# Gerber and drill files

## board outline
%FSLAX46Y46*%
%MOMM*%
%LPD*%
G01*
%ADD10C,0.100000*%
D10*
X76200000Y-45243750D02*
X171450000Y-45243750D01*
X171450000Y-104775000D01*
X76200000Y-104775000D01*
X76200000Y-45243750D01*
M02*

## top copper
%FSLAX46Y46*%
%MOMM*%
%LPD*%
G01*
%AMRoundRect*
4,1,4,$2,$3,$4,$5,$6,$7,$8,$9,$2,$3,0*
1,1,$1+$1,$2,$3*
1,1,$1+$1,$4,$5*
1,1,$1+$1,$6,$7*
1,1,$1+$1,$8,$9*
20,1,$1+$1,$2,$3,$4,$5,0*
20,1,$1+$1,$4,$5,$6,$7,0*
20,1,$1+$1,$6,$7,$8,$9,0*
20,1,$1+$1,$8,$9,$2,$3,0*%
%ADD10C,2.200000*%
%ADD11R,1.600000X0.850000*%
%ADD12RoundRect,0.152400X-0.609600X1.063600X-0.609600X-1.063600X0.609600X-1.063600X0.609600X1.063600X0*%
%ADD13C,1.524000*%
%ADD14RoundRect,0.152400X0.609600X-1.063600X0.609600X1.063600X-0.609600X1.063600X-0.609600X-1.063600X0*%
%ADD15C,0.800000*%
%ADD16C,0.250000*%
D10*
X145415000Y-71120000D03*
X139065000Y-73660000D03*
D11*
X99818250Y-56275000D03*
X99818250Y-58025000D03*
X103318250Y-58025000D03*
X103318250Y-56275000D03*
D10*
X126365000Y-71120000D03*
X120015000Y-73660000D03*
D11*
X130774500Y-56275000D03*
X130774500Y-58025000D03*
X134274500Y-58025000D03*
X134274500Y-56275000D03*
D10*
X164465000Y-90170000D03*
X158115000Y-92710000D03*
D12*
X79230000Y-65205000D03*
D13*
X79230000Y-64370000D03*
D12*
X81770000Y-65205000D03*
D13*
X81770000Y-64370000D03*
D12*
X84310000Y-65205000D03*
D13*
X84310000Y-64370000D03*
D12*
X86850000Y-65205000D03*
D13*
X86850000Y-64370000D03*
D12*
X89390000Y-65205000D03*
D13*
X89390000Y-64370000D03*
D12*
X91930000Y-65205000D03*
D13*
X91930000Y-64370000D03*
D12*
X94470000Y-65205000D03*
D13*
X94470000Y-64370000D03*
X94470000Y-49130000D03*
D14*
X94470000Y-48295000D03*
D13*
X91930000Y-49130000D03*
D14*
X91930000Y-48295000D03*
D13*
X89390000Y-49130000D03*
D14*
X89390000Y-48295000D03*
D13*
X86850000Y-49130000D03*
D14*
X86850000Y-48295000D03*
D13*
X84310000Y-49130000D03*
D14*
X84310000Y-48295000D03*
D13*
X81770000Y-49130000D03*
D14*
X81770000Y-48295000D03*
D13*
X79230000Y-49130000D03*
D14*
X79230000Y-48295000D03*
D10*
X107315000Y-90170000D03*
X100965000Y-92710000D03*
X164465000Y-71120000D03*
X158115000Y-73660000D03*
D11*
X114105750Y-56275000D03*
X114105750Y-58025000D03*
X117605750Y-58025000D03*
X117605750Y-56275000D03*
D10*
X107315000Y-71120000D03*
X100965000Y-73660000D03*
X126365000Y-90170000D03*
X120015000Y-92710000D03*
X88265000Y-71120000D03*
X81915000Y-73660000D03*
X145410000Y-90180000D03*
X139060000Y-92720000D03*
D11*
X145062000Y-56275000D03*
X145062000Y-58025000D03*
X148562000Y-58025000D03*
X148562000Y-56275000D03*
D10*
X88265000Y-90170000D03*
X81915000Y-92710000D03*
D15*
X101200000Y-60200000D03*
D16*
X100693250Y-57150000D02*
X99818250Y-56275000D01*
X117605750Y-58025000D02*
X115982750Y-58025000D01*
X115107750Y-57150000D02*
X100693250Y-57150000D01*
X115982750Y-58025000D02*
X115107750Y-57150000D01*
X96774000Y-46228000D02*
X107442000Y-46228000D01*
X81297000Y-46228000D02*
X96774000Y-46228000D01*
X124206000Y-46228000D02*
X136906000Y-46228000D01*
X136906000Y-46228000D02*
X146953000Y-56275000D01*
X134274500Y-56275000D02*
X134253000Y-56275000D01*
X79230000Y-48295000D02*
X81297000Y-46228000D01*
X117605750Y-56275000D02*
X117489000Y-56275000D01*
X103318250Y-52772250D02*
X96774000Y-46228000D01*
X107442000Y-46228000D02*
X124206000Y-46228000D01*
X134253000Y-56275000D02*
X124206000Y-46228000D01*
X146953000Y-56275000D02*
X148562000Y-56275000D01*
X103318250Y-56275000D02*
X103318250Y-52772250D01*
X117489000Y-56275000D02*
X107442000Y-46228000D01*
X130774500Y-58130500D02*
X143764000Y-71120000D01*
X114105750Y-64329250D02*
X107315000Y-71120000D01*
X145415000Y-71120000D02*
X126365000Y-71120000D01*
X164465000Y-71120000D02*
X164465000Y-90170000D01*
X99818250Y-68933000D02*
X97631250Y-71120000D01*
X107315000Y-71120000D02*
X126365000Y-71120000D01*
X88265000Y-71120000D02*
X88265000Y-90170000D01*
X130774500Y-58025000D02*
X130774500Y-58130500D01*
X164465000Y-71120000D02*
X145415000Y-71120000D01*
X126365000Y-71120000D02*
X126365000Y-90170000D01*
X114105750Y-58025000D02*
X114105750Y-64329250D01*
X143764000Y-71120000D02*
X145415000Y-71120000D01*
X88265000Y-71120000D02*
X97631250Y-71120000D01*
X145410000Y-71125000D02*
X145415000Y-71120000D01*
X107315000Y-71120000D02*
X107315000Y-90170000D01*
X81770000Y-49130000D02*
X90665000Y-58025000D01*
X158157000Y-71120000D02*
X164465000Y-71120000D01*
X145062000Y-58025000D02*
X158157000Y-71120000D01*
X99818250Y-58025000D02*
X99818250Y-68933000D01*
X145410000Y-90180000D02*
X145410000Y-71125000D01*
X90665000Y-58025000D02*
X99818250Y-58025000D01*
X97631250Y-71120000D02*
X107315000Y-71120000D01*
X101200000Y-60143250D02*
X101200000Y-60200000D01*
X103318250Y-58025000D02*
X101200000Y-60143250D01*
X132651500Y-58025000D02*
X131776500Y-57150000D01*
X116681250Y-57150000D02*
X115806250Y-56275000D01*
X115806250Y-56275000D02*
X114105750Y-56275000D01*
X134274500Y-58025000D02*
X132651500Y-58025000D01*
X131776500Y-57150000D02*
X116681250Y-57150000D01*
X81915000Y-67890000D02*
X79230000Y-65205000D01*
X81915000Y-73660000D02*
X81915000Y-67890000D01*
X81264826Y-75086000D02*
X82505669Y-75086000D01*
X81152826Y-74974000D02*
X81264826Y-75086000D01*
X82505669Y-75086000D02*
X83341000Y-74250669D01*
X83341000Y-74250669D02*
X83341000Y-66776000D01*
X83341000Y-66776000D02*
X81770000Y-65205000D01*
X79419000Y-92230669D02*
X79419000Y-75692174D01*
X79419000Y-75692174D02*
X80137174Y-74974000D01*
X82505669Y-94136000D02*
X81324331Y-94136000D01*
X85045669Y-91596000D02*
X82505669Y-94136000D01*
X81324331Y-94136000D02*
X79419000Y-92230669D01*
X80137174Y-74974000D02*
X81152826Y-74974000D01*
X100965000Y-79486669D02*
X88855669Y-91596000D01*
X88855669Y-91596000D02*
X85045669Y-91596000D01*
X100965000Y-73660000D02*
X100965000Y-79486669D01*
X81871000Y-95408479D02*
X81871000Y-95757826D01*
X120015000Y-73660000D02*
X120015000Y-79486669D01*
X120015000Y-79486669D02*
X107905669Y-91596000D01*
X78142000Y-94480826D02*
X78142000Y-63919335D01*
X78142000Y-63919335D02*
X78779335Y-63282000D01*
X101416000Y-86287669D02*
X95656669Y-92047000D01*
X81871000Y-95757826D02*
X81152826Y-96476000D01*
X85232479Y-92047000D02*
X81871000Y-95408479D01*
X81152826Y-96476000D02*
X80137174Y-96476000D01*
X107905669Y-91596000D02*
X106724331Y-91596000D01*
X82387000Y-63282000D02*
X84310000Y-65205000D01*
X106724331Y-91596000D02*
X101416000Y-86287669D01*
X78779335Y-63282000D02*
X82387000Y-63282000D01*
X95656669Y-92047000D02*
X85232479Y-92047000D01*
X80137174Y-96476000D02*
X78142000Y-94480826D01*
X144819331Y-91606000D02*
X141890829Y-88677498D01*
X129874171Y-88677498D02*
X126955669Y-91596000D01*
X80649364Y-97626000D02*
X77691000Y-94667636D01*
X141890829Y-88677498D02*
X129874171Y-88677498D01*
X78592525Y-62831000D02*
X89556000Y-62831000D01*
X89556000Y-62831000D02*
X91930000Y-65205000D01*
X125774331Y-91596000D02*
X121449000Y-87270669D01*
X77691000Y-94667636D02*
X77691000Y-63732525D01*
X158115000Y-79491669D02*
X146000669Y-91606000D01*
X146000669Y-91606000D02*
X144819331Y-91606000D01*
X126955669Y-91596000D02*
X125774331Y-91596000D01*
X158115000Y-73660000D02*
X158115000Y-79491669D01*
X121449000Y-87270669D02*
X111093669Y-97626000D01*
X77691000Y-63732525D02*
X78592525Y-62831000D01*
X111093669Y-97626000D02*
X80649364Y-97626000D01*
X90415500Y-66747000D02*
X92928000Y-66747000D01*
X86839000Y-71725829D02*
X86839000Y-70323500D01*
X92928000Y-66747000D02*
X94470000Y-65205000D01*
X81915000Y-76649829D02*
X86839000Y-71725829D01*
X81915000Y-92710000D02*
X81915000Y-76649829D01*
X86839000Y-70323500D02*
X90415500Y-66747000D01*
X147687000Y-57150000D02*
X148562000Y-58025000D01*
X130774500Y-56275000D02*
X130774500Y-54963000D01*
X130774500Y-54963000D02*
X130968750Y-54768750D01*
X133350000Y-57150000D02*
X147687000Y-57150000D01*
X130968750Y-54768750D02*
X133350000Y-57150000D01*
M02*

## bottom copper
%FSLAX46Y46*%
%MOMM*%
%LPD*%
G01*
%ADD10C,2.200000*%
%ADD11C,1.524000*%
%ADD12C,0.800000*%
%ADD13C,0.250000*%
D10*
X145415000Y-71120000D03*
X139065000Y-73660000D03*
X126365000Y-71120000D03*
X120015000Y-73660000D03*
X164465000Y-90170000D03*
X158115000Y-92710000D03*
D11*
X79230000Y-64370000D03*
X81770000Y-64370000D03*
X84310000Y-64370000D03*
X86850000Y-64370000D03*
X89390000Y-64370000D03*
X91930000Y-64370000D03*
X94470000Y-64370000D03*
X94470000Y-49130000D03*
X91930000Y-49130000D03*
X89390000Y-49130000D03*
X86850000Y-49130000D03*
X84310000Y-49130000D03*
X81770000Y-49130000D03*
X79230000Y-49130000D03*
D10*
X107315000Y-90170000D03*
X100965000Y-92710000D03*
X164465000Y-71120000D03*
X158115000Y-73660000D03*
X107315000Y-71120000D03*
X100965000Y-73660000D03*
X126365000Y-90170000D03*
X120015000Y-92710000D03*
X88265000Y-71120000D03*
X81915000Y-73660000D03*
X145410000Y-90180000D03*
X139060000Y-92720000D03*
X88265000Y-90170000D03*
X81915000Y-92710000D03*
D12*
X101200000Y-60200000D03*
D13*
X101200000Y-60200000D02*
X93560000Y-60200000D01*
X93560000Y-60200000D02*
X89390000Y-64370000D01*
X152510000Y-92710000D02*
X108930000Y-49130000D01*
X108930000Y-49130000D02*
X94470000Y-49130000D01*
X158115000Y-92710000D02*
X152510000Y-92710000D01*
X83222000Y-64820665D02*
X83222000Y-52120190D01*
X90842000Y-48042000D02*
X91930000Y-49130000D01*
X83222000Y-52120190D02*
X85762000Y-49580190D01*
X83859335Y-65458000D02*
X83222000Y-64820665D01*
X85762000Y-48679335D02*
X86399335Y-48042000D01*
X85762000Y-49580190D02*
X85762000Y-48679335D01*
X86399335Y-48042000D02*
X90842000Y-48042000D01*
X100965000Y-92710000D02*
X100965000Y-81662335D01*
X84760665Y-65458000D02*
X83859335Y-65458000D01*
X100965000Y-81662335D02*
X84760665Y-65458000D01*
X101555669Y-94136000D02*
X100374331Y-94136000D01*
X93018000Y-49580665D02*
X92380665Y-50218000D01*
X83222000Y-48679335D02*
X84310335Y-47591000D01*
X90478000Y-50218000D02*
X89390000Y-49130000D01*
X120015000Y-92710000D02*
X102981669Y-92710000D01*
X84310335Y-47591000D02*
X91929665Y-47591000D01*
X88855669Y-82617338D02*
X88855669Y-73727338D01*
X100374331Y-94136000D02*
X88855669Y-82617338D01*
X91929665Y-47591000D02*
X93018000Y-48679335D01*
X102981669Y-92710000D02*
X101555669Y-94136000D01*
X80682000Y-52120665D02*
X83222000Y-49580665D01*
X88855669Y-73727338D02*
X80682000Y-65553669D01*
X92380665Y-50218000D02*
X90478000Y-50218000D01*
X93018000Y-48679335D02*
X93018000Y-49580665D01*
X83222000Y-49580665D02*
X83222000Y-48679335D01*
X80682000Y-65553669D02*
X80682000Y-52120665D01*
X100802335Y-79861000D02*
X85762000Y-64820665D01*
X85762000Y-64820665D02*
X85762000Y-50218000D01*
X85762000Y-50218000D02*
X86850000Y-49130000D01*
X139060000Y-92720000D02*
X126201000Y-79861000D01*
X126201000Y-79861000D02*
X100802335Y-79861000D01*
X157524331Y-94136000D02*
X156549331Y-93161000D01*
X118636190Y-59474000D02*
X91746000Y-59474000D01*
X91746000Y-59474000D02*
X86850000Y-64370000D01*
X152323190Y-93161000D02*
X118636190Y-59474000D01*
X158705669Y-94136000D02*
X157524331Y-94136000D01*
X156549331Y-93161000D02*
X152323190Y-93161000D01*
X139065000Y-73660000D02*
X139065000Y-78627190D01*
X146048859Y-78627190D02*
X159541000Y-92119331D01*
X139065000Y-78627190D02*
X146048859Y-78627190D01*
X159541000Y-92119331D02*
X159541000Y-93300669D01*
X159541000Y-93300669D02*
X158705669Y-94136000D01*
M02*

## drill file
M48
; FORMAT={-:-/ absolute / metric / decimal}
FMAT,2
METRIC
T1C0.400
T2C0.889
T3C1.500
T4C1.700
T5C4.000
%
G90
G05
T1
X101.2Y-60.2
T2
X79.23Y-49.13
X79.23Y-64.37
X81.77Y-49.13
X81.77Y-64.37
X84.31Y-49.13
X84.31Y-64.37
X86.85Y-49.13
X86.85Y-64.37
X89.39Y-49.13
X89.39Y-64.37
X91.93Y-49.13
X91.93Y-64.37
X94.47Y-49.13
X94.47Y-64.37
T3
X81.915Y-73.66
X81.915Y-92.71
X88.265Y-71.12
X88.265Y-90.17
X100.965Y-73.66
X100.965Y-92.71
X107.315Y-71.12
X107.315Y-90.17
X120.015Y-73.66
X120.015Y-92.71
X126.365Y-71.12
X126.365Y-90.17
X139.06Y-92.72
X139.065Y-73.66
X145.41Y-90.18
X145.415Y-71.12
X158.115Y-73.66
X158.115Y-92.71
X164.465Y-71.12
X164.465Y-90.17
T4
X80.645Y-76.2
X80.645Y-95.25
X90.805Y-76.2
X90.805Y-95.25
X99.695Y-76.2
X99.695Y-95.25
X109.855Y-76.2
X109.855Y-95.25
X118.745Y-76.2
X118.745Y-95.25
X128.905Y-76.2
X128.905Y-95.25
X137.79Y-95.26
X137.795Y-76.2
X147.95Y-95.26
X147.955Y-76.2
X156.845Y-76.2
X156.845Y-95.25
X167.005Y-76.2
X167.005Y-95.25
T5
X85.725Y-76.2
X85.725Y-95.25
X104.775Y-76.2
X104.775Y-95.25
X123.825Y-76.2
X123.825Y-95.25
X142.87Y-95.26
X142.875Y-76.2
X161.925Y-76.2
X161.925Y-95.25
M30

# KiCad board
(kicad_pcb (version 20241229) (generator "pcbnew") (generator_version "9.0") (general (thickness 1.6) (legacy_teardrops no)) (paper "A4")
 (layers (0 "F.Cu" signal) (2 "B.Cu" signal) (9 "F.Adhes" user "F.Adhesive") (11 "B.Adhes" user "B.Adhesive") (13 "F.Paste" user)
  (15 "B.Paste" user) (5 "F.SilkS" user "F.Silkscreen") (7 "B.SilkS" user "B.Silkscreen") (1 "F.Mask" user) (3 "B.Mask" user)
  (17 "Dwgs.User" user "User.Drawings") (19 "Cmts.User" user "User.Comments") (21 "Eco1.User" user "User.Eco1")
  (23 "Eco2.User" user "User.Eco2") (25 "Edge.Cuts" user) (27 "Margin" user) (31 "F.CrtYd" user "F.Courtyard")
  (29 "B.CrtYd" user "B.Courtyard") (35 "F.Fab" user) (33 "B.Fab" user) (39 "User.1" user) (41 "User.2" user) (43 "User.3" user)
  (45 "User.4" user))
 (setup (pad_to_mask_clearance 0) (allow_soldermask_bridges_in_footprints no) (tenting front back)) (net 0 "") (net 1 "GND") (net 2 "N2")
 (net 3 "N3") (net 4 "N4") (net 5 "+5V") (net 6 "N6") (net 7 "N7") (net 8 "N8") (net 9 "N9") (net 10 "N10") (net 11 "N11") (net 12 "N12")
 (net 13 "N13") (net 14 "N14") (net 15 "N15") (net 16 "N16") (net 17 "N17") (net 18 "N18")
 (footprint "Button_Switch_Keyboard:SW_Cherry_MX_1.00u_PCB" (layer "F.Cu") (at 145.415 71.12)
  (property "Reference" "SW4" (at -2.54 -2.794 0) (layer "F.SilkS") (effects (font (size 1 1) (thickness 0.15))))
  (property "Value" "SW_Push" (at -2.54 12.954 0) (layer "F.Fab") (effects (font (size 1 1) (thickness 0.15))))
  (pad "" np_thru_hole circle (at -7.62 5.08) (size 1.7 1.7) (drill 1.7) (layers "*.Cu" "*.Mask"))
  (pad "" np_thru_hole circle (at -2.54 5.08) (size 4 4) (drill 4) (layers "*.Cu" "*.Mask"))
  (pad "" np_thru_hole circle (at 2.54 5.08) (size 1.7 1.7) (drill 1.7) (layers "*.Cu" "*.Mask"))
  (pad "1" thru_hole circle (at 0 0) (size 2.2 2.2) (drill 1.5) (layers "*.Cu" "*.Mask") (remove_unused_layers no) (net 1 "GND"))
  (pad "2" thru_hole circle (at -6.35 2.54) (size 2.2 2.2) (drill 1.5) (layers "*.Cu" "*.Mask") (remove_unused_layers no) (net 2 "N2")))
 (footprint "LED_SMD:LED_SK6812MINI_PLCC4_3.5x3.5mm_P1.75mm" (layer "F.Cu") (at 101.56825 57.15)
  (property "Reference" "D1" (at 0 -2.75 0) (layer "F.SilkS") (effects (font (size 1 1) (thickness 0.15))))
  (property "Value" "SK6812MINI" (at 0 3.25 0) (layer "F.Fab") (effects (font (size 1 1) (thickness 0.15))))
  (pad "1" smd rect (at -1.75 -0.875) (size 1.6 0.85) (layers "F.Cu" "F.Mask" "F.Paste") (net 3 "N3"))
  (pad "2" smd rect (at -1.75 0.875) (size 1.6 0.85) (layers "F.Cu" "F.Mask" "F.Paste") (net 1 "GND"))
  (pad "3" smd rect (at 1.75 0.875) (size 1.6 0.85) (layers "F.Cu" "F.Mask" "F.Paste") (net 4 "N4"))
  (pad "4" smd rect (at 1.75 -0.875) (size 1.6 0.85) (layers "F.Cu" "F.Mask" "F.Paste") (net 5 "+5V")))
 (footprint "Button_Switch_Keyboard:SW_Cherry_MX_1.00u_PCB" (layer "F.Cu") (at 126.365 71.12)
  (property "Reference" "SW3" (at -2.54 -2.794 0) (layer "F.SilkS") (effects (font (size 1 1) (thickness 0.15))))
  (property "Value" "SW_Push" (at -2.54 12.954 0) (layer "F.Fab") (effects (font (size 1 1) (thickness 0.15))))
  (pad "" np_thru_hole circle (at -7.62 5.08) (size 1.7 1.7) (drill 1.7) (layers "*.Cu" "*.Mask"))
  (pad "" np_thru_hole circle (at -2.54 5.08) (size 4 4) (drill 4) (layers "*.Cu" "*.Mask"))
  (pad "" np_thru_hole circle (at 2.54 5.08) (size 1.7 1.7) (drill 1.7) (layers "*.Cu" "*.Mask"))
  (pad "1" thru_hole circle (at 0 0) (size 2.2 2.2) (drill 1.5) (layers "*.Cu" "*.Mask") (remove_unused_layers no) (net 1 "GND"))
  (pad "2" thru_hole circle (at -6.35 2.54) (size 2.2 2.2) (drill 1.5) (layers "*.Cu" "*.Mask") (remove_unused_layers no) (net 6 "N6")))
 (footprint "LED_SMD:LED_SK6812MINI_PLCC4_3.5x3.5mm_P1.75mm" (layer "F.Cu") (at 132.5245 57.15)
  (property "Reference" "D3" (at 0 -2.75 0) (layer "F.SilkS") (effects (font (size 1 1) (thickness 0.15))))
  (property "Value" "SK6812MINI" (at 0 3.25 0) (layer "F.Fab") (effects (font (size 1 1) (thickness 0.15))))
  (pad "1" smd rect (at -1.75 -0.875) (size 1.6 0.85) (layers "F.Cu" "F.Mask" "F.Paste") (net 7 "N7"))
  (pad "2" smd rect (at -1.75 0.875) (size 1.6 0.85) (layers "F.Cu" "F.Mask" "F.Paste") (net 1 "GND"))
  (pad "3" smd rect (at 1.75 0.875) (size 1.6 0.85) (layers "F.Cu" "F.Mask" "F.Paste") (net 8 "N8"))
  (pad "4" smd rect (at 1.75 -0.875) (size 1.6 0.85) (layers "F.Cu" "F.Mask" "F.Paste") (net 5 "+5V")))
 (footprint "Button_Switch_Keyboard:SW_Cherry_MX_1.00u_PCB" (layer "F.Cu") (at 164.465 90.17)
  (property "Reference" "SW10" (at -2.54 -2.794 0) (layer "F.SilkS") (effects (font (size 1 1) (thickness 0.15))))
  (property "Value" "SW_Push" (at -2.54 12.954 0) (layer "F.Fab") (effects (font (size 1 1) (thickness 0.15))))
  (pad "" np_thru_hole circle (at -7.62 5.08) (size 1.7 1.7) (drill 1.7) (layers "*.Cu" "*.Mask"))
  (pad "" np_thru_hole circle (at -2.54 5.08) (size 4 4) (drill 4) (layers "*.Cu" "*.Mask"))
  (pad "" np_thru_hole circle (at 2.54 5.08) (size 1.7 1.7) (drill 1.7) (layers "*.Cu" "*.Mask"))
  (pad "1" thru_hole circle (at 0 0) (size 2.2 2.2) (drill 1.5) (layers "*.Cu" "*.Mask") (remove_unused_layers no) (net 1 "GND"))
  (pad "2" thru_hole circle (at -6.35 2.54) (size 2.2 2.2) (drill 1.5) (layers "*.Cu" "*.Mask") (remove_unused_layers no) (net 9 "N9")))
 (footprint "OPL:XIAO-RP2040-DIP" (layer "F.Cu") (at 86.85 56.75 90)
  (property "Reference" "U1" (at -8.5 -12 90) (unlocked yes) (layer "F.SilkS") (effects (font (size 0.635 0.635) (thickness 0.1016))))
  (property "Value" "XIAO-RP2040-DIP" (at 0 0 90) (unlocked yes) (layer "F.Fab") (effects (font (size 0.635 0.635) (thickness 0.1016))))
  (pad "1" smd roundrect (at -8.455 -7.62 270) (size 2.432 1.524) (layers "F.Cu" "F.Mask") (roundrect_rratio 0.1) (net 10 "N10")
   (thermal_bridge_angle 45))
  (pad "1" thru_hole circle (at -7.62 -7.62 270) (size 1.524 1.524) (drill 0.889) (layers "*.Cu" "*.Mask") (remove_unused_layers no)
   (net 10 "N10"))
  (pad "2" smd roundrect (at -8.455 -5.08 270) (size 2.432 1.524) (layers "F.Cu" "F.Mask") (roundrect_rratio 0.1) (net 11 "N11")
   (thermal_bridge_angle 45))
  (pad "2" thru_hole circle (at -7.62 -5.08 270) (size 1.524 1.524) (drill 0.889) (layers "*.Cu" "*.Mask") (remove_unused_layers no)
   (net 11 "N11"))
  (pad "3" smd roundrect (at -8.455 -2.54 270) (size 2.432 1.524) (layers "F.Cu" "F.Mask") (roundrect_rratio 0.1) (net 6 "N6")
   (thermal_bridge_angle 45))
  (pad "3" thru_hole circle (at -7.62 -2.54 270) (size 1.524 1.524) (drill 0.889) (layers "*.Cu" "*.Mask") (remove_unused_layers no)
   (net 6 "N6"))
  (pad "4" smd roundrect (at -8.455 0 270) (size 2.432 1.524) (layers "F.Cu" "F.Mask") (roundrect_rratio 0.1) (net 2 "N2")
   (thermal_bridge_angle 45))
  (pad "4" thru_hole circle (at -7.62 0 270) (size 1.524 1.524) (drill 0.889) (layers "*.Cu" "*.Mask") (remove_unused_layers no)
   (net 2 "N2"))
  (pad "5" smd roundrect (at -8.455 2.54 270) (size 2.432 1.524) (layers "F.Cu" "F.Mask") (roundrect_rratio 0.1) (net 4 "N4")
   (thermal_bridge_angle 45))
  (pad "5" thru_hole circle (at -7.62 2.54 270) (size 1.524 1.524) (drill 0.889) (layers "*.Cu" "*.Mask") (remove_unused_layers no)
   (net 4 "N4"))
  (pad "6" smd roundrect (at -8.455 5.08 270) (size 2.432 1.524) (layers "F.Cu" "F.Mask") (roundrect_rratio 0.1) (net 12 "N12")
   (thermal_bridge_angle 45))
  (pad "6" thru_hole circle (at -7.62 5.08 270) (size 1.524 1.524) (drill 0.889) (layers "*.Cu" "*.Mask") (remove_unused_layers no)
   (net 12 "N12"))
  (pad "7" smd roundrect (at -8.455 7.62 270) (size 2.432 1.524) (layers "F.Cu" "F.Mask") (roundrect_rratio 0.1) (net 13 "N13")
   (thermal_bridge_angle 45))
  (pad "7" thru_hole circle (at -7.62 7.62 270) (size 1.524 1.524) (drill 0.889) (layers "*.Cu" "*.Mask") (remove_unused_layers no)
   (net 13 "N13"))
  (pad "8" thru_hole circle (at 7.62 7.62 90) (size 1.524 1.524) (drill 0.889) (layers "*.Cu" "*.Mask") (remove_unused_layers no)
   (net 9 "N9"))
  (pad "8" smd roundrect (at 8.455 7.62 90) (size 2.432 1.524) (layers "F.Cu" "F.Mask") (roundrect_rratio 0.1) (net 9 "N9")
   (thermal_bridge_angle 45))
  (pad "9" thru_hole circle (at 7.62 5.08 90) (size 1.524 1.524) (drill 0.889) (layers "*.Cu" "*.Mask") (remove_unused_layers no)
   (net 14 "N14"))
  (pad "9" smd roundrect (at 8.455 5.08 90) (size 2.432 1.524) (layers "F.Cu" "F.Mask") (roundrect_rratio 0.1) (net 14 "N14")
   (thermal_bridge_angle 45))
  (pad "10" thru_hole circle (at 7.62 2.54 90) (size 1.524 1.524) (drill 0.889) (layers "*.Cu" "*.Mask") (remove_unused_layers no)
   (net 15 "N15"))
  (pad "10" smd roundrect (at 8.455 2.54 90) (size 2.432 1.524) (layers "F.Cu" "F.Mask") (roundrect_rratio 0.1) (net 15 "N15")
   (thermal_bridge_angle 45))
  (pad "11" thru_hole circle (at 7.62 0 90) (size 1.524 1.524) (drill 0.889) (layers "*.Cu" "*.Mask") (remove_unused_layers no)
   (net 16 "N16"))
  (pad "11" smd roundrect (at 8.455 0 90) (size 2.432 1.524) (layers "F.Cu" "F.Mask") (roundrect_rratio 0.1) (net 16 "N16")
   (thermal_bridge_angle 45))
  (pad "12" thru_hole circle (at 7.62 -2.54 90) (size 1.524 1.524) (drill 0.889) (layers "*.Cu" "*.Mask") (remove_unused_layers no)
   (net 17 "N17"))
  (pad "12" smd roundrect (at 8.455 -2.54 90) (size 2.432 1.524) (layers "F.Cu" "F.Mask") (roundrect_rratio 0.1) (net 17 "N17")
   (thermal_bridge_angle 45))
  (pad "13" thru_hole circle (at 7.62 -5.08 90) (size 1.524 1.524) (drill 0.889) (layers "*.Cu" "*.Mask") (remove_unused_layers no)
   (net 1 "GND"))
  (pad "13" smd roundrect (at 8.455 -5.08 90) (size 2.432 1.524) (layers "F.Cu" "F.Mask") (roundrect_rratio 0.1) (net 1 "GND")
   (thermal_bridge_angle 45))
  (pad "14" thru_hole circle (at 7.62 -7.62 90) (size 1.524 1.524) (drill 0.889) (layers "*.Cu" "*.Mask") (remove_unused_layers no)
   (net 5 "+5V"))
  (pad "14" smd roundrect (at 8.455 -7.62 90) (size 2.432 1.524) (layers "F.Cu" "F.Mask") (roundrect_rratio 0.1) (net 5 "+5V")
   (thermal_bridge_angle 45)))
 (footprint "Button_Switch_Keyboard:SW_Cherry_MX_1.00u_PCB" (layer "F.Cu") (at 107.315 90.17)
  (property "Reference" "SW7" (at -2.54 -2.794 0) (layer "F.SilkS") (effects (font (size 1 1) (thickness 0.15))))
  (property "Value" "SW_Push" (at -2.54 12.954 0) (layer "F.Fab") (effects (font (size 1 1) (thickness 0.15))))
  (pad "" np_thru_hole circle (at -7.62 5.08) (size 1.7 1.7) (drill 1.7) (layers "*.Cu" "*.Mask"))
  (pad "" np_thru_hole circle (at -2.54 5.08) (size 4 4) (drill 4) (layers "*.Cu" "*.Mask"))
  (pad "" np_thru_hole circle (at 2.54 5.08) (size 1.7 1.7) (drill 1.7) (layers "*.Cu" "*.Mask"))
  (pad "1" thru_hole circle (at 0 0) (size 2.2 2.2) (drill 1.5) (layers "*.Cu" "*.Mask") (remove_unused_layers no) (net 1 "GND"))
  (pad "2" thru_hole circle (at -6.35 2.54) (size 2.2 2.2) (drill 1.5) (layers "*.Cu" "*.Mask") (remove_unused_layers no) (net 14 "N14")))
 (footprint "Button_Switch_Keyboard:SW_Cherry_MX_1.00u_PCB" (layer "F.Cu") (at 164.465 71.12)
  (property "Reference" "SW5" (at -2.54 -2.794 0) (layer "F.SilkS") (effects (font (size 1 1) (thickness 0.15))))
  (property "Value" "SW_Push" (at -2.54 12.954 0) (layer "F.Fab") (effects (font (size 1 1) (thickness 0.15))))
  (pad "" np_thru_hole circle (at -7.62 5.08) (size 1.7 1.7) (drill 1.7) (layers "*.Cu" "*.Mask"))
  (pad "" np_thru_hole circle (at -2.54 5.08) (size 4 4) (drill 4) (layers "*.Cu" "*.Mask"))
  (pad "" np_thru_hole circle (at 2.54 5.08) (size 1.7 1.7) (drill 1.7) (layers "*.Cu" "*.Mask"))
  (pad "1" thru_hole circle (at 0 0) (size 2.2 2.2) (drill 1.5) (layers "*.Cu" "*.Mask") (remove_unused_layers no) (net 1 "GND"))
  (pad "2" thru_hole circle (at -6.35 2.54) (size 2.2 2.2) (drill 1.5) (layers "*.Cu" "*.Mask") (remove_unused_layers no) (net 12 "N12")))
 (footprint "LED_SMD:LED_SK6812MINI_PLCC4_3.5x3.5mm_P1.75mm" (layer "F.Cu") (at 115.85575 57.15)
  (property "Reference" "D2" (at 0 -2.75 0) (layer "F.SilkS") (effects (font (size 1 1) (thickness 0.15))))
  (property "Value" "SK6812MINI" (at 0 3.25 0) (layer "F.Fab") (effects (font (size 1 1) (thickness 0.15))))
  (pad "1" smd rect (at -1.75 -0.875) (size 1.6 0.85) (layers "F.Cu" "F.Mask" "F.Paste") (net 8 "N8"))
  (pad "2" smd rect (at -1.75 0.875) (size 1.6 0.85) (layers "F.Cu" "F.Mask" "F.Paste") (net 1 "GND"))
  (pad "3" smd rect (at 1.75 0.875) (size 1.6 0.85) (layers "F.Cu" "F.Mask" "F.Paste") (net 3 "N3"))
  (pad "4" smd rect (at 1.75 -0.875) (size 1.6 0.85) (layers "F.Cu" "F.Mask" "F.Paste") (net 5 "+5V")))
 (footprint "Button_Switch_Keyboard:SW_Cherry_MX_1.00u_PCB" (layer "F.Cu") (at 107.315 71.12)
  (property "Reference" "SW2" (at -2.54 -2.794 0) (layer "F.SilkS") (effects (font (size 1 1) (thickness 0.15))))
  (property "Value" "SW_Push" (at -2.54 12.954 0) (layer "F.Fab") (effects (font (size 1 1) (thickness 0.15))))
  (pad "" np_thru_hole circle (at -7.62 5.08) (size 1.7 1.7) (drill 1.7) (layers "*.Cu" "*.Mask"))
  (pad "" np_thru_hole circle (at -2.54 5.08) (size 4 4) (drill 4) (layers "*.Cu" "*.Mask"))
  (pad "" np_thru_hole circle (at 2.54 5.08) (size 1.7 1.7) (drill 1.7) (layers "*.Cu" "*.Mask"))
  (pad "1" thru_hole circle (at 0 0) (size 2.2 2.2) (drill 1.5) (layers "*.Cu" "*.Mask") (remove_unused_layers no) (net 1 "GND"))
  (pad "2" thru_hole circle (at -6.35 2.54) (size 2.2 2.2) (drill 1.5) (layers "*.Cu" "*.Mask") (remove_unused_layers no) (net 11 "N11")))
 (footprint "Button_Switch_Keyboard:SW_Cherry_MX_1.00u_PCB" (layer "F.Cu") (at 126.365 90.17)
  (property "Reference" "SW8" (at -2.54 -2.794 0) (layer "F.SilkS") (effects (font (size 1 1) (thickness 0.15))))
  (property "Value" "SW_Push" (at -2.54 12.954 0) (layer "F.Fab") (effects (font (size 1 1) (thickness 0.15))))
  (pad "" np_thru_hole circle (at -7.62 5.08) (size 1.7 1.7) (drill 1.7) (layers "*.Cu" "*.Mask"))
  (pad "" np_thru_hole circle (at -2.54 5.08) (size 4 4) (drill 4) (layers "*.Cu" "*.Mask"))
  (pad "" np_thru_hole circle (at 2.54 5.08) (size 1.7 1.7) (drill 1.7) (layers "*.Cu" "*.Mask"))
  (pad "1" thru_hole circle (at 0 0) (size 2.2 2.2) (drill 1.5) (layers "*.Cu" "*.Mask") (remove_unused_layers no) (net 1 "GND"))
  (pad "2" thru_hole circle (at -6.35 2.54) (size 2.2 2.2) (drill 1.5) (layers "*.Cu" "*.Mask") (remove_unused_layers no) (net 15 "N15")))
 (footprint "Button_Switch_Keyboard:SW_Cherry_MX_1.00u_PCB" (layer "F.Cu") (at 88.265 71.12)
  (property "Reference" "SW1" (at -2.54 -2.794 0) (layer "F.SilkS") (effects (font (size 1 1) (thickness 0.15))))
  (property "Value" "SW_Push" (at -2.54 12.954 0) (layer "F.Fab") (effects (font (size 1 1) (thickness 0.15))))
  (pad "" np_thru_hole circle (at -7.62 5.08) (size 1.7 1.7) (drill 1.7) (layers "*.Cu" "*.Mask"))
  (pad "" np_thru_hole circle (at -2.54 5.08) (size 4 4) (drill 4) (layers "*.Cu" "*.Mask"))
  (pad "" np_thru_hole circle (at 2.54 5.08) (size 1.7 1.7) (drill 1.7) (layers "*.Cu" "*.Mask"))
  (pad "1" thru_hole circle (at 0 0) (size 2.2 2.2) (drill 1.5) (layers "*.Cu" "*.Mask") (remove_unused_layers no) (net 1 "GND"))
  (pad "2" thru_hole circle (at -6.35 2.54) (size 2.2 2.2) (drill 1.5) (layers "*.Cu" "*.Mask") (remove_unused_layers no) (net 10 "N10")))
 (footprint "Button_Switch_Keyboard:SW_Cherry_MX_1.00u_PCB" (layer "F.Cu") (at 145.41 90.18)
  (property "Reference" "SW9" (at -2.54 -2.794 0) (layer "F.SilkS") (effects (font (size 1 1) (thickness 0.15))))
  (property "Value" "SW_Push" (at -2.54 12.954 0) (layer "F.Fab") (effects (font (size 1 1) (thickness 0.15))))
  (pad "" np_thru_hole circle (at -7.62 5.08) (size 1.7 1.7) (drill 1.7) (layers "*.Cu" "*.Mask"))
  (pad "" np_thru_hole circle (at -2.54 5.08) (size 4 4) (drill 4) (layers "*.Cu" "*.Mask"))
  (pad "" np_thru_hole circle (at 2.54 5.08) (size 1.7 1.7) (drill 1.7) (layers "*.Cu" "*.Mask"))
  (pad "1" thru_hole circle (at 0 0) (size 2.2 2.2) (drill 1.5) (layers "*.Cu" "*.Mask") (remove_unused_layers no) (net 1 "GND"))
  (pad "2" thru_hole circle (at -6.35 2.54) (size 2.2 2.2) (drill 1.5) (layers "*.Cu" "*.Mask") (remove_unused_layers no) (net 16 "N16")))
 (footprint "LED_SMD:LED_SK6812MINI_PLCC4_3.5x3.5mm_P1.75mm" (layer "F.Cu") (at 146.812 57.15)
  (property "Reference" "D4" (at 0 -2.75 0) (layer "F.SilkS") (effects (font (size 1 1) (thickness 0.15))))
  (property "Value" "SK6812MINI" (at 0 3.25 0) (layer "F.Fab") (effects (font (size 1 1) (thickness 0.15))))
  (pad "1" smd rect (at -1.75 -0.875) (size 1.6 0.85) (layers "F.Cu" "F.Mask" "F.Paste") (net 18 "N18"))
  (pad "2" smd rect (at -1.75 0.875) (size 1.6 0.85) (layers "F.Cu" "F.Mask" "F.Paste") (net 1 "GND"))
  (pad "3" smd rect (at 1.75 0.875) (size 1.6 0.85) (layers "F.Cu" "F.Mask" "F.Paste") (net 7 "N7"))
  (pad "4" smd rect (at 1.75 -0.875) (size 1.6 0.85) (layers "F.Cu" "F.Mask" "F.Paste") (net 5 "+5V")))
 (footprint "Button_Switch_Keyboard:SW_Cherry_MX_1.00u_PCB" (layer "F.Cu") (at 88.265 90.17)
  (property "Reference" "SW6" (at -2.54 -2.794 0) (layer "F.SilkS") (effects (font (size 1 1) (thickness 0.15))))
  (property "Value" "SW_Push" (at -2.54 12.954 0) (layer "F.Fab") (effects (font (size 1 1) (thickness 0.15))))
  (pad "" np_thru_hole circle (at -7.62 5.08) (size 1.7 1.7) (drill 1.7) (layers "*.Cu" "*.Mask"))
  (pad "" np_thru_hole circle (at -2.54 5.08) (size 4 4) (drill 4) (layers "*.Cu" "*.Mask"))
  (pad "" np_thru_hole circle (at 2.54 5.08) (size 1.7 1.7) (drill 1.7) (layers "*.Cu" "*.Mask"))
  (pad "1" thru_hole circle (at 0 0) (size 2.2 2.2) (drill 1.5) (layers "*.Cu" "*.Mask") (remove_unused_layers no) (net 1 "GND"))
  (pad "2" thru_hole circle (at -6.35 2.54) (size 2.2 2.2) (drill 1.5) (layers "*.Cu" "*.Mask") (remove_unused_layers no) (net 13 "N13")))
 (gr_rect (start 76.2 45.24375) (end 171.45 104.775) (stroke (width 0.1) (type default)) (fill no) (layer "Edge.Cuts"))
 (segment (start 100.69325 57.15) (end 99.81825 56.275) (width 0.25) (layer "F.Cu") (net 3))
 (segment (start 117.60575 58.025) (end 115.98275 58.025) (width 0.25) (layer "F.Cu") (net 3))
 (segment (start 115.10775 57.15) (end 100.69325 57.15) (width 0.25) (layer "F.Cu") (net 3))
 (segment (start 115.98275 58.025) (end 115.10775 57.15) (width 0.25) (layer "F.Cu") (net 3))
 (segment (start 96.774 46.228) (end 107.442 46.228) (width 0.25) (layer "F.Cu") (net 5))
 (segment (start 81.297 46.228) (end 96.774 46.228) (width 0.25) (layer "F.Cu") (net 5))
 (segment (start 124.206 46.228) (end 136.906 46.228) (width 0.25) (layer "F.Cu") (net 5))
 (segment (start 136.906 46.228) (end 146.953 56.275) (width 0.25) (layer "F.Cu") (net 5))
 (segment (start 134.2745 56.275) (end 134.253 56.275) (width 0.25) (layer "F.Cu") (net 5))
 (segment (start 79.23 48.295) (end 81.297 46.228) (width 0.25) (layer "F.Cu") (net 5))
 (segment (start 117.60575 56.275) (end 117.489 56.275) (width 0.25) (layer "F.Cu") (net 5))
 (segment (start 103.31825 52.77225) (end 96.774 46.228) (width 0.25) (layer "F.Cu") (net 5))
 (segment (start 107.442 46.228) (end 124.206 46.228) (width 0.25) (layer "F.Cu") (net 5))
 (segment (start 134.253 56.275) (end 124.206 46.228) (width 0.25) (layer "F.Cu") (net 5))
 (segment (start 146.953 56.275) (end 148.562 56.275) (width 0.25) (layer "F.Cu") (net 5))
 (segment (start 103.31825 56.275) (end 103.31825 52.77225) (width 0.25) (layer "F.Cu") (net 5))
 (segment (start 117.489 56.275) (end 107.442 46.228) (width 0.25) (layer "F.Cu") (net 5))
 (segment (start 130.7745 58.1305) (end 143.764 71.12) (width 0.25) (layer "F.Cu") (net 1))
 (segment (start 114.10575 64.32925) (end 107.315 71.12) (width 0.25) (layer "F.Cu") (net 1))
 (segment (start 145.415 71.12) (end 126.365 71.12) (width 0.25) (layer "F.Cu") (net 1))
 (segment (start 164.465 71.12) (end 164.465 90.17) (width 0.25) (layer "F.Cu") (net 1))
 (segment (start 99.81825 68.933) (end 97.63125 71.12) (width 0.25) (layer "F.Cu") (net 1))
 (segment (start 107.315 71.12) (end 126.365 71.12) (width 0.25) (layer "F.Cu") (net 1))
 (segment (start 88.265 71.12) (end 88.265 90.17) (width 0.25) (layer "F.Cu") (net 1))
 (segment (start 130.7745 58.025) (end 130.7745 58.1305) (width 0.25) (layer "F.Cu") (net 1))
 (segment (start 164.465 71.12) (end 145.415 71.12) (width 0.25) (layer "F.Cu") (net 1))
 (segment (start 126.365 71.12) (end 126.365 90.17) (width 0.25) (layer "F.Cu") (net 1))
 (segment (start 114.10575 58.025) (end 114.10575 64.32925) (width 0.25) (layer "F.Cu") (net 1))
 (segment (start 143.764 71.12) (end 145.415 71.12) (width 0.25) (layer "F.Cu") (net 1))
 (segment (start 88.265 71.12) (end 97.63125 71.12) (width 0.25) (layer "F.Cu") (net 1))
 (segment (start 145.41 71.125) (end 145.415 71.12) (width 0.25) (layer "F.Cu") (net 1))
 (segment (start 107.315 71.12) (end 107.315 90.17) (width 0.25) (layer "F.Cu") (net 1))
 (segment (start 81.77 49.13) (end 90.665 58.025) (width 0.25) (layer "F.Cu") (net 1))
 (segment (start 158.157 71.12) (end 164.465 71.12) (width 0.25) (layer "F.Cu") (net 1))
 (segment (start 145.062 58.025) (end 158.157 71.12) (width 0.25) (layer "F.Cu") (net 1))
 (segment (start 99.81825 58.025) (end 99.81825 68.933) (width 0.25) (layer "F.Cu") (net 1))
 (segment (start 145.41 90.18) (end 145.41 71.125) (width 0.25) (layer "F.Cu") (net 1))
 (segment (start 90.665 58.025) (end 99.81825 58.025) (width 0.25) (layer "F.Cu") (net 1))
 (segment (start 97.63125 71.12) (end 107.315 71.12) (width 0.25) (layer "F.Cu") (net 1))
 (segment (start 101.2 60.14325) (end 101.2 60.2) (width 0.25) (layer "F.Cu") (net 4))
 (segment (start 103.31825 58.025) (end 101.2 60.14325) (width 0.25) (layer "F.Cu") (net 4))
 (via (at 101.2 60.2) (size 0.8) (drill 0.4) (layers "F.Cu" "B.Cu") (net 4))
 (segment (start 101.2 60.2) (end 93.56 60.2) (width 0.25) (layer "B.Cu") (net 4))
 (segment (start 93.56 60.2) (end 89.39 64.37) (width 0.25) (layer "B.Cu") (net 4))
 (segment (start 132.6515 58.025) (end 131.7765 57.15) (width 0.25) (layer "F.Cu") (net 8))
 (segment (start 116.68125 57.15) (end 115.80625 56.275) (width 0.25) (layer "F.Cu") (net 8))
 (segment (start 115.80625 56.275) (end 114.10575 56.275) (width 0.25) (layer "F.Cu") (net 8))
 (segment (start 134.2745 58.025) (end 132.6515 58.025) (width 0.25) (layer "F.Cu") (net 8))
 (segment (start 131.7765 57.15) (end 116.68125 57.15) (width 0.25) (layer "F.Cu") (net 8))
 (segment (start 152.51 92.71) (end 108.93 49.13) (width 0.25) (layer "B.Cu") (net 9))
 (segment (start 108.93 49.13) (end 94.47 49.13) (width 0.25) (layer "B.Cu") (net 9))
 (segment (start 158.115 92.71) (end 152.51 92.71) (width 0.25) (layer "B.Cu") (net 9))
 (segment (start 83.222 64.820665) (end 83.222 52.12019) (width 0.25) (layer "B.Cu") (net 14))
 (segment (start 90.842 48.042) (end 91.93 49.13) (width 0.25) (layer "B.Cu") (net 14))
 (segment (start 83.222 52.12019) (end 85.762 49.58019) (width 0.25) (layer "B.Cu") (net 14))
 (segment (start 83.859335 65.458) (end 83.222 64.820665) (width 0.25) (layer "B.Cu") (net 14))
 (segment (start 85.762 48.679335) (end 86.399335 48.042) (width 0.25) (layer "B.Cu") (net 14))
 (segment (start 85.762 49.58019) (end 85.762 48.679335) (width 0.25) (layer "B.Cu") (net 14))
 (segment (start 86.399335 48.042) (end 90.842 48.042) (width 0.25) (layer "B.Cu") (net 14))
 (segment (start 100.965 92.71) (end 100.965 81.662335) (width 0.25) (layer "B.Cu") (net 14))
 (segment (start 84.760665 65.458) (end 83.859335 65.458) (width 0.25) (layer "B.Cu") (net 14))
 (segment (start 100.965 81.662335) (end 84.760665 65.458) (width 0.25) (layer "B.Cu") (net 14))
 (segment (start 101.555669 94.136) (end 100.374331 94.136) (width 0.25) (layer "B.Cu") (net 15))
 (segment (start 93.018 49.580665) (end 92.380665 50.218) (width 0.25) (layer "B.Cu") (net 15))
 (segment (start 83.222 48.679335) (end 84.310335 47.591) (width 0.25) (layer "B.Cu") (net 15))
 (segment (start 90.478 50.218) (end 89.39 49.13) (width 0.25) (layer "B.Cu") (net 15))
 (segment (start 120.015 92.71) (end 102.981669 92.71) (width 0.25) (layer "B.Cu") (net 15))
 (segment (start 84.310335 47.591) (end 91.929665 47.591) (width 0.25) (layer "B.Cu") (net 15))
 (segment (start 88.855669 82.617338) (end 88.855669 73.727338) (width 0.25) (layer "B.Cu") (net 15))
 (segment (start 100.374331 94.136) (end 88.855669 82.617338) (width 0.25) (layer "B.Cu") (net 15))
 (segment (start 91.929665 47.591) (end 93.018 48.679335) (width 0.25) (layer "B.Cu") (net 15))
 (segment (start 102.981669 92.71) (end 101.555669 94.136) (width 0.25) (layer "B.Cu") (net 15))
 (segment (start 80.682 52.120665) (end 83.222 49.580665) (width 0.25) (layer "B.Cu") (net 15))
 (segment (start 88.855669 73.727338) (end 80.682 65.553669) (width 0.25) (layer "B.Cu") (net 15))
 (segment (start 92.380665 50.218) (end 90.478 50.218) (width 0.25) (layer "B.Cu") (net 15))
 (segment (start 93.018 48.679335) (end 93.018 49.580665) (width 0.25) (layer "B.Cu") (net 15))
 (segment (start 83.222 49.580665) (end 83.222 48.679335) (width 0.25) (layer "B.Cu") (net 15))
 (segment (start 80.682 65.553669) (end 80.682 52.120665) (width 0.25) (layer "B.Cu") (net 15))
 (segment (start 100.802335 79.861) (end 85.762 64.820665) (width 0.25) (layer "B.Cu") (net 16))
 (segment (start 85.762 64.820665) (end 85.762 50.218) (width 0.25) (layer "B.Cu") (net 16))
 (segment (start 85.762 50.218) (end 86.85 49.13) (width 0.25) (layer "B.Cu") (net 16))
 (segment (start 139.06 92.72) (end 126.201 79.861) (width 0.25) (layer "B.Cu") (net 16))
 (segment (start 126.201 79.861) (end 100.802335 79.861) (width 0.25) (layer "B.Cu") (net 16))
 (segment (start 81.915 67.89) (end 79.23 65.205) (width 0.25) (layer "F.Cu") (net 10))
 (segment (start 81.915 73.66) (end 81.915 67.89) (width 0.25) (layer "F.Cu") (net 10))
 (segment (start 81.264826 75.086) (end 82.505669 75.086) (width 0.25) (layer "F.Cu") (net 11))
 (segment (start 81.152826 74.974) (end 81.264826 75.086) (width 0.25) (layer "F.Cu") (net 11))
 (segment (start 82.505669 75.086) (end 83.341 74.250669) (width 0.25) (layer "F.Cu") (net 11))
 (segment (start 83.341 74.250669) (end 83.341 66.776) (width 0.25) (layer "F.Cu") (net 11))
 (segment (start 83.341 66.776) (end 81.77 65.205) (width 0.25) (layer "F.Cu") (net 11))
 (segment (start 79.419 92.230669) (end 79.419 75.692174) (width 0.25) (layer "F.Cu") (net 11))
 (segment (start 79.419 75.692174) (end 80.137174 74.974) (width 0.25) (layer "F.Cu") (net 11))
 (segment (start 82.505669 94.136) (end 81.324331 94.136) (width 0.25) (layer "F.Cu") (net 11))
 (segment (start 85.045669 91.596) (end 82.505669 94.136) (width 0.25) (layer "F.Cu") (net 11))
 (segment (start 81.324331 94.136) (end 79.419 92.230669) (width 0.25) (layer "F.Cu") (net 11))
 (segment (start 80.137174 74.974) (end 81.152826 74.974) (width 0.25) (layer "F.Cu") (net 11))
 (segment (start 100.965 79.486669) (end 88.855669 91.596) (width 0.25) (layer "F.Cu") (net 11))
 (segment (start 88.855669 91.596) (end 85.045669 91.596) (width 0.25) (layer "F.Cu") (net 11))
 (segment (start 100.965 73.66) (end 100.965 79.486669) (width 0.25) (layer "F.Cu") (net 11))
 (segment (start 81.871 95.408479) (end 81.871 95.757826) (width 0.25) (layer "F.Cu") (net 6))
 (segment (start 120.015 73.66) (end 120.015 79.486669) (width 0.25) (layer "F.Cu") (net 6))
 (segment (start 120.015 79.486669) (end 107.905669 91.596) (width 0.25) (layer "F.Cu") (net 6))
 (segment (start 78.142 94.480826) (end 78.142 63.919335) (width 0.25) (layer "F.Cu") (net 6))
 (segment (start 78.142 63.919335) (end 78.779335 63.282) (width 0.25) (layer "F.Cu") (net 6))
 (segment (start 101.416 86.287669) (end 95.656669 92.047) (width 0.25) (layer "F.Cu") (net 6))
 (segment (start 81.871 95.757826) (end 81.152826 96.476) (width 0.25) (layer "F.Cu") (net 6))
 (segment (start 85.232479 92.047) (end 81.871 95.408479) (width 0.25) (layer "F.Cu") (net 6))
 (segment (start 81.152826 96.476) (end 80.137174 96.476) (width 0.25) (layer "F.Cu") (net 6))
 (segment (start 107.905669 91.596) (end 106.724331 91.596) (width 0.25) (layer "F.Cu") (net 6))
 (segment (start 82.387 63.282) (end 84.31 65.205) (width 0.25) (layer "F.Cu") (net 6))
 (segment (start 106.724331 91.596) (end 101.416 86.287669) (width 0.25) (layer "F.Cu") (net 6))
 (segment (start 78.779335 63.282) (end 82.387 63.282) (width 0.25) (layer "F.Cu") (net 6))
 (segment (start 95.656669 92.047) (end 85.232479 92.047) (width 0.25) (layer "F.Cu") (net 6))
 (segment (start 80.137174 96.476) (end 78.142 94.480826) (width 0.25) (layer "F.Cu") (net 6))
 (segment (start 157.524331 94.136) (end 156.549331 93.161) (width 0.25) (layer "B.Cu") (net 2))
 (segment (start 118.63619 59.474) (end 91.746 59.474) (width 0.25) (layer "B.Cu") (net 2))
 (segment (start 91.746 59.474) (end 86.85 64.37) (width 0.25) (layer "B.Cu") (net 2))
 (segment (start 152.32319 93.161) (end 118.63619 59.474) (width 0.25) (layer "B.Cu") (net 2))
 (segment (start 158.705669 94.136) (end 157.524331 94.136) (width 0.25) (layer "B.Cu") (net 2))
 (segment (start 156.549331 93.161) (end 152.32319 93.161) (width 0.25) (layer "B.Cu") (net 2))
 (segment (start 139.065 73.66) (end 139.065 78.62719) (width 0.25) (layer "B.Cu") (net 2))
 (segment (start 146.048859 78.62719) (end 159.541 92.119331) (width 0.25) (layer "B.Cu") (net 2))
 (segment (start 139.065 78.62719) (end 146.048859 78.62719) (width 0.25) (layer "B.Cu") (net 2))
 (segment (start 159.541 92.119331) (end 159.541 93.300669) (width 0.25) (layer "B.Cu") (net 2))
 (segment (start 159.541 93.300669) (end 158.705669 94.136) (width 0.25) (layer "B.Cu") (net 2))
 (segment (start 144.819331 91.606) (end 141.890829 88.677498) (width 0.25) (layer "F.Cu") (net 12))
 (segment (start 129.874171 88.677498) (end 126.955669 91.596) (width 0.25) (layer "F.Cu") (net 12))
 (segment (start 80.649364 97.626) (end 77.691 94.667636) (width 0.25) (layer "F.Cu") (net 12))
 (segment (start 141.890829 88.677498) (end 129.874171 88.677498) (width 0.25) (layer "F.Cu") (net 12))
 (segment (start 78.592525 62.831) (end 89.556 62.831) (width 0.25) (layer "F.Cu") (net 12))
 (segment (start 89.556 62.831) (end 91.93 65.205) (width 0.25) (layer "F.Cu") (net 12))
 (segment (start 125.774331 91.596) (end 121.449 87.270669) (width 0.25) (layer "F.Cu") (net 12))
 (segment (start 77.691 94.667636) (end 77.691 63.732525) (width 0.25) (layer "F.Cu") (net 12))
 (segment (start 158.115 79.491669) (end 146.000669 91.606) (width 0.25) (layer "F.Cu") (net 12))
 (segment (start 146.000669 91.606) (end 144.819331 91.606) (width 0.25) (layer "F.Cu") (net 12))
 (segment (start 126.955669 91.596) (end 125.774331 91.596) (width 0.25) (layer "F.Cu") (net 12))
 (segment (start 158.115 73.66) (end 158.115 79.491669) (width 0.25) (layer "F.Cu") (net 12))
 (segment (start 121.449 87.270669) (end 111.093669 97.626) (width 0.25) (layer "F.Cu") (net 12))
 (segment (start 77.691 63.732525) (end 78.592525 62.831) (width 0.25) (layer "F.Cu") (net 12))
 (segment (start 111.093669 97.626) (end 80.649364 97.626) (width 0.25) (layer "F.Cu") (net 12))
 (segment (start 90.4155 66.747) (end 92.928 66.747) (width 0.25) (layer "F.Cu") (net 13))
 (segment (start 86.839 71.725829) (end 86.839 70.3235) (width 0.25) (layer "F.Cu") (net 13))
 (segment (start 92.928 66.747) (end 94.47 65.205) (width 0.25) (layer "F.Cu") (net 13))
 (segment (start 81.915 76.649829) (end 86.839 71.725829) (width 0.25) (layer "F.Cu") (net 13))
 (segment (start 81.915 92.71) (end 81.915 76.649829) (width 0.25) (layer "F.Cu") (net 13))
 (segment (start 86.839 70.3235) (end 90.4155 66.747) (width 0.25) (layer "F.Cu") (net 13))
 (segment (start 147.687 57.15) (end 148.562 58.025) (width 0.25) (layer "F.Cu") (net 7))
 (segment (start 130.7745 56.275) (end 130.7745 54.963) (width 0.25) (layer "F.Cu") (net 7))
 (segment (start 130.7745 54.963) (end 130.96875 54.76875) (width 0.25) (layer "F.Cu") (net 7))
 (segment (start 133.35 57.15) (end 147.687 57.15) (width 0.25) (layer "F.Cu") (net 7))
 (segment (start 130.96875 54.76875) (end 133.35 57.15) (width 0.25) (layer "F.Cu") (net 7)))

